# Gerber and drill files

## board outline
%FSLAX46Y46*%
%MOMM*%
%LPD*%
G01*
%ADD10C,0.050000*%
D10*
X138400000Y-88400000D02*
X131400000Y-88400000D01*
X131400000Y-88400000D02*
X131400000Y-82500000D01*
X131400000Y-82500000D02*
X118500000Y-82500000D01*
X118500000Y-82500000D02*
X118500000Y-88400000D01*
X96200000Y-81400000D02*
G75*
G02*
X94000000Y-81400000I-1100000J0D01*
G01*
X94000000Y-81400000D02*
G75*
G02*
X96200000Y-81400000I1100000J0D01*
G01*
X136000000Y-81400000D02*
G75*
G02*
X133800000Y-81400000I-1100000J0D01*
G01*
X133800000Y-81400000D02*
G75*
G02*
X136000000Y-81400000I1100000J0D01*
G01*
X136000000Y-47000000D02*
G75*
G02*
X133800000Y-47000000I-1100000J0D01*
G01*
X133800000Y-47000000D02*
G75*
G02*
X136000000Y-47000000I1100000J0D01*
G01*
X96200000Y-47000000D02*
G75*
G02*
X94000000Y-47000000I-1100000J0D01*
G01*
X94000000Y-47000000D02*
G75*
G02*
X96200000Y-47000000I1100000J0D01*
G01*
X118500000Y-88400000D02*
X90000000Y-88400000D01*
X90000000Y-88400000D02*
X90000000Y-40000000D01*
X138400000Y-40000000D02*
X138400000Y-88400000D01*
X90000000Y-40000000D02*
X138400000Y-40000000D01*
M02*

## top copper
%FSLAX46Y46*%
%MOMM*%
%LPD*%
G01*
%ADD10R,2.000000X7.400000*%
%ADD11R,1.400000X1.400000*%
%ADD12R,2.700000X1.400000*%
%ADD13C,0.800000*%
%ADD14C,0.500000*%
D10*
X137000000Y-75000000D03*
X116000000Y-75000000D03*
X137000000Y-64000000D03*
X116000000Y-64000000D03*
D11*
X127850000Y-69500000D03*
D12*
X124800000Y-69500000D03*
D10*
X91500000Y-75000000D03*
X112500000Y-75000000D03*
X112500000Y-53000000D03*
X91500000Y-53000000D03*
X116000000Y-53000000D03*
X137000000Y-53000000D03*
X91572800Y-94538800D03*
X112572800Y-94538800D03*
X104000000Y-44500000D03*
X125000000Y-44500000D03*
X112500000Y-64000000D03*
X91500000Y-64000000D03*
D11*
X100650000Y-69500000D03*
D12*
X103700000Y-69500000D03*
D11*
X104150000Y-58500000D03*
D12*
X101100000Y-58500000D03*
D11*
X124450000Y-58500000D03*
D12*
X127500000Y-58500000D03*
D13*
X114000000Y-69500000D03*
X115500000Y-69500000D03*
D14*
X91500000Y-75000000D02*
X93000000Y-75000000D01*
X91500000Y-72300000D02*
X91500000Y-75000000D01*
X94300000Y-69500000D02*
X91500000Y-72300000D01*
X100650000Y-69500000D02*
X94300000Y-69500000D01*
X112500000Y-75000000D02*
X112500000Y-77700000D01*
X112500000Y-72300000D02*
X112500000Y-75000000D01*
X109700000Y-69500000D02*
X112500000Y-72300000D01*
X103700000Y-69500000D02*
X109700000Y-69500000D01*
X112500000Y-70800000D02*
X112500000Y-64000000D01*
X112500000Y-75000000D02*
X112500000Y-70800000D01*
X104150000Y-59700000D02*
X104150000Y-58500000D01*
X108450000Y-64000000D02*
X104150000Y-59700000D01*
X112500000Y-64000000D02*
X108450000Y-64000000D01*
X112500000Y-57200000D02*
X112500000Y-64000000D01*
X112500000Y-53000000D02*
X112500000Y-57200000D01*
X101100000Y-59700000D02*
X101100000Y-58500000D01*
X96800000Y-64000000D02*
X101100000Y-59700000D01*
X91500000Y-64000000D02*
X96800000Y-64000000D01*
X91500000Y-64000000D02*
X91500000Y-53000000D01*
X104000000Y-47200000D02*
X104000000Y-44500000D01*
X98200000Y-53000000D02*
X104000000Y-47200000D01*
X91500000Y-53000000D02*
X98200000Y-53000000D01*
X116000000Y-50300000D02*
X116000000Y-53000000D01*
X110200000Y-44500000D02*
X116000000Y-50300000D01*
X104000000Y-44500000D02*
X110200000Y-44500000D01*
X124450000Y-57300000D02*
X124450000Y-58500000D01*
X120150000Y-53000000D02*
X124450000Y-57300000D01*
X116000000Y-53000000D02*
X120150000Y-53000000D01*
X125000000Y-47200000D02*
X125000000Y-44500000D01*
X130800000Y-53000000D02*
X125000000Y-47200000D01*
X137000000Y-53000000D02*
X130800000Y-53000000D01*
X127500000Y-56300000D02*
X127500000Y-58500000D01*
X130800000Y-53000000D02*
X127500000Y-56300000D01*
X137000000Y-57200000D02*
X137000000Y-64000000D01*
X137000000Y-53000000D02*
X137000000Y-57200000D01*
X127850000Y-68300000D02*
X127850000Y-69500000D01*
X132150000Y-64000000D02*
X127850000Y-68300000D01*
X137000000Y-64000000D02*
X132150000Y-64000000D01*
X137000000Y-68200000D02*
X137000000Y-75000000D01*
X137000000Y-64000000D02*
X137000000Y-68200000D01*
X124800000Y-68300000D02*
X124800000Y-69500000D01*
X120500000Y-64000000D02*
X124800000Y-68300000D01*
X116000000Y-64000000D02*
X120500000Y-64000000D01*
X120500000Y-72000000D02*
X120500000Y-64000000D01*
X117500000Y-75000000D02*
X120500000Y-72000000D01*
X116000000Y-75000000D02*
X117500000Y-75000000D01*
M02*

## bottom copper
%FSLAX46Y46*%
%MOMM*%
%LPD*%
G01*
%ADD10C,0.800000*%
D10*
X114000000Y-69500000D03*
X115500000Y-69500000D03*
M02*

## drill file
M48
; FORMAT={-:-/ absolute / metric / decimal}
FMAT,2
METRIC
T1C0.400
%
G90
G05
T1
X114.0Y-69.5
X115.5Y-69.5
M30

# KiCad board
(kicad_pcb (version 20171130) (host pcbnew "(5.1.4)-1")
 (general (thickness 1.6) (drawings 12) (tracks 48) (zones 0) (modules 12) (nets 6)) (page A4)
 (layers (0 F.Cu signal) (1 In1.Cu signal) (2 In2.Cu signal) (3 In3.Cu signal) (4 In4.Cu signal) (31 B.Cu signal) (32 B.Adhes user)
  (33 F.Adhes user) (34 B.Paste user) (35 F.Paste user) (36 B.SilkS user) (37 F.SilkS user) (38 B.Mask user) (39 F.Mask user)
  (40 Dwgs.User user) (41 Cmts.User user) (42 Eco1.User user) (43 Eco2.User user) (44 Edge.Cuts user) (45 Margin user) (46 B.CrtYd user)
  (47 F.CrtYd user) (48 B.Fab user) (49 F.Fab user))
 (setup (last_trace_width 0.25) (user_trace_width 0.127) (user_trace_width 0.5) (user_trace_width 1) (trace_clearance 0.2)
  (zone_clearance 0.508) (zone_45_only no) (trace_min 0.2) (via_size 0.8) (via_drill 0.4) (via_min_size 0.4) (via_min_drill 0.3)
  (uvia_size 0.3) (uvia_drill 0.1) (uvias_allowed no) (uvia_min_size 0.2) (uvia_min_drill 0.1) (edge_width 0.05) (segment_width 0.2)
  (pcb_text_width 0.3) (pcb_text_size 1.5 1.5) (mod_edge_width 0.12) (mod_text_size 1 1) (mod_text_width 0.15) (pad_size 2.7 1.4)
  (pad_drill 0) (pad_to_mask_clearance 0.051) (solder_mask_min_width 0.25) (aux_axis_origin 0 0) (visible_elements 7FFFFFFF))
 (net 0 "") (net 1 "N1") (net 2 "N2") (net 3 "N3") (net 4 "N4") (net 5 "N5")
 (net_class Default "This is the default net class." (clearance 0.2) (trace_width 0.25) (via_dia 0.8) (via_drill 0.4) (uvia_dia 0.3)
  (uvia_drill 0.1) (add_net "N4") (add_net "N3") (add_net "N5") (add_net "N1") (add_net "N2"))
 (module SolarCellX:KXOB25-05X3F (layer F.Cu) (at 116 75)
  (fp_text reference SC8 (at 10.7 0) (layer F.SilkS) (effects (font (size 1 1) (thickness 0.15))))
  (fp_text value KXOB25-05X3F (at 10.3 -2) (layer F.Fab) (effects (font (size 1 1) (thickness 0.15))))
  (pad 2 smd rect (at 21 0) (size 2 7.4) (layers F.Cu F.Paste F.Mask) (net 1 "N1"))
  (pad 1 smd rect (at 0 0) (size 2 7.4) (layers F.Cu F.Paste F.Mask) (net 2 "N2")))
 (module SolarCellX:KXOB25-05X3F (layer F.Cu) (at 116 64)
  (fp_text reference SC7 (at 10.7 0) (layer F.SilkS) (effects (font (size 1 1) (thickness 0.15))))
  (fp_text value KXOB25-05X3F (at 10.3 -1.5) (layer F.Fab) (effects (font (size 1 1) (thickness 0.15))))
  (pad 2 smd rect (at 21 0) (size 2 7.4) (layers F.Cu F.Paste F.Mask) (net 1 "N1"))
  (pad 1 smd rect (at 0 0) (size 2 7.4) (layers F.Cu F.Paste F.Mask) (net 2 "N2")))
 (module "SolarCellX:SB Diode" (layer F.Cu) (at 126 69.5)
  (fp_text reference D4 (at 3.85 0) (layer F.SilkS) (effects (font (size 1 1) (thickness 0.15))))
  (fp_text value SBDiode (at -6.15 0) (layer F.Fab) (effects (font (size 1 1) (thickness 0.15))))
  (pad 2 smd rect (at 1.85 0) (size 1.4 1.4) (layers F.Cu F.Paste F.Mask) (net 1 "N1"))
  (pad 1 smd rect (at -1.2 0) (size 2.7 1.4) (layers F.Cu F.Paste F.Mask) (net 2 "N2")))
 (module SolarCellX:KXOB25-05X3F (layer F.Cu) (at 112.5 75 180)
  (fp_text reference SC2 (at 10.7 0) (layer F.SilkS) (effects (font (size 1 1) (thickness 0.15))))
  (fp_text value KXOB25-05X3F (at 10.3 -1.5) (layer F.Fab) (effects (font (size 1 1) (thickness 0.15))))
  (pad 2 smd rect (at 21 0 180) (size 2 7.4) (layers F.Cu F.Paste F.Mask) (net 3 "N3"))
  (pad 1 smd rect (at 0 0 180) (size 2 7.4) (layers F.Cu F.Paste F.Mask) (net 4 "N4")))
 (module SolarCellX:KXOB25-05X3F (layer F.Cu) (at 91.5 53)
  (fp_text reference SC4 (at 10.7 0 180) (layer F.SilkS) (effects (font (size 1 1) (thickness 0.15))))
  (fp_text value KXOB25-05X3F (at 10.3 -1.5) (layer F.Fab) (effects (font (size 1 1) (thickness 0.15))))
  (pad 2 smd rect (at 21 0) (size 2 7.4) (layers F.Cu F.Paste F.Mask) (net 4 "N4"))
  (pad 1 smd rect (at 0 0) (size 2 7.4) (layers F.Cu F.Paste F.Mask) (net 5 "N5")))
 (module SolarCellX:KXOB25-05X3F (layer F.Cu) (at 137 53 180)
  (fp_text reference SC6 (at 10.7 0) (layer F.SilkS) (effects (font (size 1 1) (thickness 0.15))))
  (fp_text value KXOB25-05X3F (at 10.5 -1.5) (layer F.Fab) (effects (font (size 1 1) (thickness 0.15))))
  (pad 2 smd rect (at 21 0 180) (size 2 7.4) (layers F.Cu F.Paste F.Mask) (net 5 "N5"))
  (pad 1 smd rect (at 0 0 180) (size 2 7.4) (layers F.Cu F.Paste F.Mask) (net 1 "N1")))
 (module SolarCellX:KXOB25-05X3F (layer F.Cu) (at 112.5728 94.5388 180)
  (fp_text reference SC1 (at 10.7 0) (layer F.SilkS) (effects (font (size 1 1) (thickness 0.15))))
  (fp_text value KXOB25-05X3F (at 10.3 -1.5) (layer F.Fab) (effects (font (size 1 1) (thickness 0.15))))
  (pad 2 smd rect (at 21 0 180) (size 2 7.4) (layers F.Cu F.Paste F.Mask) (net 3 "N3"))
  (pad 1 smd rect (at 0 0 180) (size 2 7.4) (layers F.Cu F.Paste F.Mask) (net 4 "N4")))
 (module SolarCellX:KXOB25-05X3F (layer F.Cu) (at 125 44.5 180)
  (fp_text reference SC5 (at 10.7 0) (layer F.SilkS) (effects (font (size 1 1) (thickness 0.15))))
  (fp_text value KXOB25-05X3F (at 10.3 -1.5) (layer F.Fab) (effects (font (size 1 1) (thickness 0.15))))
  (pad 2 smd rect (at 21 0 180) (size 2 7.4) (layers F.Cu F.Paste F.Mask) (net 5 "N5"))
  (pad 1 smd rect (at 0 0 180) (size 2 7.4) (layers F.Cu F.Paste F.Mask) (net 1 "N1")))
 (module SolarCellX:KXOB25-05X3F (layer F.Cu) (at 91.5 64)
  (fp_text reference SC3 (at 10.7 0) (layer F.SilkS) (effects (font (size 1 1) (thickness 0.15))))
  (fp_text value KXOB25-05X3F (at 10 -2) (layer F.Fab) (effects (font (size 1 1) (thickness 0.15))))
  (pad 2 smd rect (at 21 0) (size 2 7.4) (layers F.Cu F.Paste F.Mask) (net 4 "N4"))
  (pad 1 smd rect (at 0 0) (size 2 7.4) (layers F.Cu F.Paste F.Mask) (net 5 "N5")))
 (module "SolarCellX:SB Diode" (layer F.Cu) (at 102.5 69.5 180)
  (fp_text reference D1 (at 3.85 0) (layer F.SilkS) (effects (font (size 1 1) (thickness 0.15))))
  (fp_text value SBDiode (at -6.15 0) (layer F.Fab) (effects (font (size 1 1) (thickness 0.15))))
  (pad 2 smd rect (at 1.85 0 180) (size 1.4 1.4) (layers F.Cu F.Paste F.Mask) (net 3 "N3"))
  (pad 1 smd rect (at -1.2 0 180) (size 2.7 1.4) (layers F.Cu F.Paste F.Mask) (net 4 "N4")))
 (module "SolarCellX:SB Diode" (layer F.Cu) (at 102.3 58.5)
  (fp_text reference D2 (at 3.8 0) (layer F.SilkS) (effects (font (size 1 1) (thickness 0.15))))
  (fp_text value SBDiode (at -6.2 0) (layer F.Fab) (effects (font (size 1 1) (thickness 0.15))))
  (pad 2 smd rect (at 1.85 0) (size 1.4 1.4) (layers F.Cu F.Paste F.Mask) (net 4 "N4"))
  (pad 1 smd rect (at -1.2 0) (size 2.7 1.4) (layers F.Cu F.Paste F.Mask) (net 5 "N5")))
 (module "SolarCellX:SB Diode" (layer F.Cu) (at 126.3 58.5 180)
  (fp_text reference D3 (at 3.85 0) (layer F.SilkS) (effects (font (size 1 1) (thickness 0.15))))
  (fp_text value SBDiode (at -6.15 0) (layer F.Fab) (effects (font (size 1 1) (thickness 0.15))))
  (pad 2 smd rect (at 1.85 0 180) (size 1.4 1.4) (layers F.Cu F.Paste F.Mask) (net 5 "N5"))
  (pad 1 smd rect (at -1.2 0 180) (size 2.7 1.4) (layers F.Cu F.Paste F.Mask) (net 1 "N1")))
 (gr_line (start 138.4 88.4) (end 131.4 88.4) (layer Edge.Cuts) (width 0.05))
 (gr_line (start 131.4 88.4) (end 131.4 82.5) (layer Edge.Cuts) (width 0.05))
 (gr_line (start 131.4 82.5) (end 118.5 82.5) (layer Edge.Cuts) (width 0.05))
 (gr_line (start 118.5 82.5) (end 118.5 88.4) (layer Edge.Cuts) (width 0.05))
 (gr_circle (center 95.1 81.4) (end 96.2 81.4) (layer Edge.Cuts) (width 0.05))
 (gr_circle (center 134.9 81.4) (end 136 81.4) (layer Edge.Cuts) (width 0.05))
 (gr_circle (center 134.9 47) (end 136 47) (layer Edge.Cuts) (width 0.05))
 (gr_circle (center 95.1 47) (end 96.2 47) (layer Edge.Cuts) (width 0.05))
 (gr_line (start 118.5 88.4) (end 90 88.4) (layer Edge.Cuts) (width 0.05))
 (gr_line (start 90 88.4) (end 90 40) (layer Edge.Cuts) (width 0.05))
 (gr_line (start 138.4 40) (end 138.4 88.4) (layer Edge.Cuts) (width 0.05))
 (gr_line (start 90 40) (end 138.4 40) (layer Edge.Cuts) (width 0.05))
 (via (at 114 69.5) (size 0.8) (drill 0.4) (layers F.Cu B.Cu) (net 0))
 (via (at 115.5 69.5) (size 0.8) (drill 0.4) (layers F.Cu B.Cu) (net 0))
 (segment (start 91.5 75) (end 93 75) (width 0.5) (layer F.Cu) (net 3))
 (segment (start 91.5 72.3) (end 91.5 75) (width 0.5) (layer F.Cu) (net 3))
 (segment (start 94.3 69.5) (end 91.5 72.3) (width 0.5) (layer F.Cu) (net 3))
 (segment (start 100.65 69.5) (end 94.3 69.5) (width 0.5) (layer F.Cu) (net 3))
 (segment (start 112.5 75) (end 112.5 77.7) (width 0.5) (layer F.Cu) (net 4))
 (segment (start 112.5 72.3) (end 112.5 75) (width 0.5) (layer F.Cu) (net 4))
 (segment (start 109.7 69.5) (end 112.5 72.3) (width 0.5) (layer F.Cu) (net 4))
 (segment (start 103.7 69.5) (end 109.7 69.5) (width 0.5) (layer F.Cu) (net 4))
 (segment (start 112.5 70.8) (end 112.5 64) (width 0.5) (layer F.Cu) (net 4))
 (segment (start 112.5 75) (end 112.5 70.8) (width 0.5) (layer F.Cu) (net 4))
 (segment (start 104.15 59.7) (end 104.15 58.5) (width 0.5) (layer F.Cu) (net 4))
 (segment (start 108.45 64) (end 104.15 59.7) (width 0.5) (layer F.Cu) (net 4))
 (segment (start 112.5 64) (end 108.45 64) (width 0.5) (layer F.Cu) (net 4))
 (segment (start 112.5 57.2) (end 112.5 64) (width 0.5) (layer F.Cu) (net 4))
 (segment (start 112.5 53) (end 112.5 57.2) (width 0.5) (layer F.Cu) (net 4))
 (segment (start 101.1 59.7) (end 101.1 58.5) (width 0.5) (layer F.Cu) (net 5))
 (segment (start 96.8 64) (end 101.1 59.7) (width 0.5) (layer F.Cu) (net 5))
 (segment (start 91.5 64) (end 96.8 64) (width 0.5) (layer F.Cu) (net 5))
 (segment (start 91.5 64) (end 91.5 53) (width 0.5) (layer F.Cu) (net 5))
 (segment (start 104 47.2) (end 104 44.5) (width 0.5) (layer F.Cu) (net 5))
 (segment (start 98.2 53) (end 104 47.2) (width 0.5) (layer F.Cu) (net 5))
 (segment (start 91.5 53) (end 98.2 53) (width 0.5) (layer F.Cu) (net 5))
 (segment (start 116 50.3) (end 116 53) (width 0.5) (layer F.Cu) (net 5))
 (segment (start 110.2 44.5) (end 116 50.3) (width 0.5) (layer F.Cu) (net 5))
 (segment (start 104 44.5) (end 110.2 44.5) (width 0.5) (layer F.Cu) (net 5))
 (segment (start 124.45 57.3) (end 124.45 58.5) (width 0.5) (layer F.Cu) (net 5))
 (segment (start 120.15 53) (end 124.45 57.3) (width 0.5) (layer F.Cu) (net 5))
 (segment (start 116 53) (end 120.15 53) (width 0.5) (layer F.Cu) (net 5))
 (segment (start 125 47.2) (end 125 44.5) (width 0.5) (layer F.Cu) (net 1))
 (segment (start 130.8 53) (end 125 47.2) (width 0.5) (layer F.Cu) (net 1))
 (segment (start 137 53) (end 130.8 53) (width 0.5) (layer F.Cu) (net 1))
 (segment (start 127.5 56.3) (end 127.5 58.5) (width 0.5) (layer F.Cu) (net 1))
 (segment (start 130.8 53) (end 127.5 56.3) (width 0.5) (layer F.Cu) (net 1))
 (segment (start 137 57.2) (end 137 64) (width 0.5) (layer F.Cu) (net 1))
 (segment (start 137 53) (end 137 57.2) (width 0.5) (layer F.Cu) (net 1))
 (segment (start 127.85 68.3) (end 127.85 69.5) (width 0.5) (layer F.Cu) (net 1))
 (segment (start 132.15 64) (end 127.85 68.3) (width 0.5) (layer F.Cu) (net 1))
 (segment (start 137 64) (end 132.15 64) (width 0.5) (layer F.Cu) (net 1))
 (segment (start 137 68.2) (end 137 75) (width 0.5) (layer F.Cu) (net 1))
 (segment (start 137 64) (end 137 68.2) (width 0.5) (layer F.Cu) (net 1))
 (segment (start 124.8 68.3) (end 124.8 69.5) (width 0.5) (layer F.Cu) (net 2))
 (segment (start 120.5 64) (end 124.8 68.3) (width 0.5) (layer F.Cu) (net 2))
 (segment (start 116 64) (end 120.5 64) (width 0.5) (layer F.Cu) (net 2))
 (segment (start 120.5 72) (end 120.5 64) (width 0.5) (layer F.Cu) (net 2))
 (segment (start 117.5 75) (end 120.5 72) (width 0.5) (layer F.Cu) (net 2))
 (segment (start 116 75) (end 117.5 75) (width 0.5) (layer F.Cu) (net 2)))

